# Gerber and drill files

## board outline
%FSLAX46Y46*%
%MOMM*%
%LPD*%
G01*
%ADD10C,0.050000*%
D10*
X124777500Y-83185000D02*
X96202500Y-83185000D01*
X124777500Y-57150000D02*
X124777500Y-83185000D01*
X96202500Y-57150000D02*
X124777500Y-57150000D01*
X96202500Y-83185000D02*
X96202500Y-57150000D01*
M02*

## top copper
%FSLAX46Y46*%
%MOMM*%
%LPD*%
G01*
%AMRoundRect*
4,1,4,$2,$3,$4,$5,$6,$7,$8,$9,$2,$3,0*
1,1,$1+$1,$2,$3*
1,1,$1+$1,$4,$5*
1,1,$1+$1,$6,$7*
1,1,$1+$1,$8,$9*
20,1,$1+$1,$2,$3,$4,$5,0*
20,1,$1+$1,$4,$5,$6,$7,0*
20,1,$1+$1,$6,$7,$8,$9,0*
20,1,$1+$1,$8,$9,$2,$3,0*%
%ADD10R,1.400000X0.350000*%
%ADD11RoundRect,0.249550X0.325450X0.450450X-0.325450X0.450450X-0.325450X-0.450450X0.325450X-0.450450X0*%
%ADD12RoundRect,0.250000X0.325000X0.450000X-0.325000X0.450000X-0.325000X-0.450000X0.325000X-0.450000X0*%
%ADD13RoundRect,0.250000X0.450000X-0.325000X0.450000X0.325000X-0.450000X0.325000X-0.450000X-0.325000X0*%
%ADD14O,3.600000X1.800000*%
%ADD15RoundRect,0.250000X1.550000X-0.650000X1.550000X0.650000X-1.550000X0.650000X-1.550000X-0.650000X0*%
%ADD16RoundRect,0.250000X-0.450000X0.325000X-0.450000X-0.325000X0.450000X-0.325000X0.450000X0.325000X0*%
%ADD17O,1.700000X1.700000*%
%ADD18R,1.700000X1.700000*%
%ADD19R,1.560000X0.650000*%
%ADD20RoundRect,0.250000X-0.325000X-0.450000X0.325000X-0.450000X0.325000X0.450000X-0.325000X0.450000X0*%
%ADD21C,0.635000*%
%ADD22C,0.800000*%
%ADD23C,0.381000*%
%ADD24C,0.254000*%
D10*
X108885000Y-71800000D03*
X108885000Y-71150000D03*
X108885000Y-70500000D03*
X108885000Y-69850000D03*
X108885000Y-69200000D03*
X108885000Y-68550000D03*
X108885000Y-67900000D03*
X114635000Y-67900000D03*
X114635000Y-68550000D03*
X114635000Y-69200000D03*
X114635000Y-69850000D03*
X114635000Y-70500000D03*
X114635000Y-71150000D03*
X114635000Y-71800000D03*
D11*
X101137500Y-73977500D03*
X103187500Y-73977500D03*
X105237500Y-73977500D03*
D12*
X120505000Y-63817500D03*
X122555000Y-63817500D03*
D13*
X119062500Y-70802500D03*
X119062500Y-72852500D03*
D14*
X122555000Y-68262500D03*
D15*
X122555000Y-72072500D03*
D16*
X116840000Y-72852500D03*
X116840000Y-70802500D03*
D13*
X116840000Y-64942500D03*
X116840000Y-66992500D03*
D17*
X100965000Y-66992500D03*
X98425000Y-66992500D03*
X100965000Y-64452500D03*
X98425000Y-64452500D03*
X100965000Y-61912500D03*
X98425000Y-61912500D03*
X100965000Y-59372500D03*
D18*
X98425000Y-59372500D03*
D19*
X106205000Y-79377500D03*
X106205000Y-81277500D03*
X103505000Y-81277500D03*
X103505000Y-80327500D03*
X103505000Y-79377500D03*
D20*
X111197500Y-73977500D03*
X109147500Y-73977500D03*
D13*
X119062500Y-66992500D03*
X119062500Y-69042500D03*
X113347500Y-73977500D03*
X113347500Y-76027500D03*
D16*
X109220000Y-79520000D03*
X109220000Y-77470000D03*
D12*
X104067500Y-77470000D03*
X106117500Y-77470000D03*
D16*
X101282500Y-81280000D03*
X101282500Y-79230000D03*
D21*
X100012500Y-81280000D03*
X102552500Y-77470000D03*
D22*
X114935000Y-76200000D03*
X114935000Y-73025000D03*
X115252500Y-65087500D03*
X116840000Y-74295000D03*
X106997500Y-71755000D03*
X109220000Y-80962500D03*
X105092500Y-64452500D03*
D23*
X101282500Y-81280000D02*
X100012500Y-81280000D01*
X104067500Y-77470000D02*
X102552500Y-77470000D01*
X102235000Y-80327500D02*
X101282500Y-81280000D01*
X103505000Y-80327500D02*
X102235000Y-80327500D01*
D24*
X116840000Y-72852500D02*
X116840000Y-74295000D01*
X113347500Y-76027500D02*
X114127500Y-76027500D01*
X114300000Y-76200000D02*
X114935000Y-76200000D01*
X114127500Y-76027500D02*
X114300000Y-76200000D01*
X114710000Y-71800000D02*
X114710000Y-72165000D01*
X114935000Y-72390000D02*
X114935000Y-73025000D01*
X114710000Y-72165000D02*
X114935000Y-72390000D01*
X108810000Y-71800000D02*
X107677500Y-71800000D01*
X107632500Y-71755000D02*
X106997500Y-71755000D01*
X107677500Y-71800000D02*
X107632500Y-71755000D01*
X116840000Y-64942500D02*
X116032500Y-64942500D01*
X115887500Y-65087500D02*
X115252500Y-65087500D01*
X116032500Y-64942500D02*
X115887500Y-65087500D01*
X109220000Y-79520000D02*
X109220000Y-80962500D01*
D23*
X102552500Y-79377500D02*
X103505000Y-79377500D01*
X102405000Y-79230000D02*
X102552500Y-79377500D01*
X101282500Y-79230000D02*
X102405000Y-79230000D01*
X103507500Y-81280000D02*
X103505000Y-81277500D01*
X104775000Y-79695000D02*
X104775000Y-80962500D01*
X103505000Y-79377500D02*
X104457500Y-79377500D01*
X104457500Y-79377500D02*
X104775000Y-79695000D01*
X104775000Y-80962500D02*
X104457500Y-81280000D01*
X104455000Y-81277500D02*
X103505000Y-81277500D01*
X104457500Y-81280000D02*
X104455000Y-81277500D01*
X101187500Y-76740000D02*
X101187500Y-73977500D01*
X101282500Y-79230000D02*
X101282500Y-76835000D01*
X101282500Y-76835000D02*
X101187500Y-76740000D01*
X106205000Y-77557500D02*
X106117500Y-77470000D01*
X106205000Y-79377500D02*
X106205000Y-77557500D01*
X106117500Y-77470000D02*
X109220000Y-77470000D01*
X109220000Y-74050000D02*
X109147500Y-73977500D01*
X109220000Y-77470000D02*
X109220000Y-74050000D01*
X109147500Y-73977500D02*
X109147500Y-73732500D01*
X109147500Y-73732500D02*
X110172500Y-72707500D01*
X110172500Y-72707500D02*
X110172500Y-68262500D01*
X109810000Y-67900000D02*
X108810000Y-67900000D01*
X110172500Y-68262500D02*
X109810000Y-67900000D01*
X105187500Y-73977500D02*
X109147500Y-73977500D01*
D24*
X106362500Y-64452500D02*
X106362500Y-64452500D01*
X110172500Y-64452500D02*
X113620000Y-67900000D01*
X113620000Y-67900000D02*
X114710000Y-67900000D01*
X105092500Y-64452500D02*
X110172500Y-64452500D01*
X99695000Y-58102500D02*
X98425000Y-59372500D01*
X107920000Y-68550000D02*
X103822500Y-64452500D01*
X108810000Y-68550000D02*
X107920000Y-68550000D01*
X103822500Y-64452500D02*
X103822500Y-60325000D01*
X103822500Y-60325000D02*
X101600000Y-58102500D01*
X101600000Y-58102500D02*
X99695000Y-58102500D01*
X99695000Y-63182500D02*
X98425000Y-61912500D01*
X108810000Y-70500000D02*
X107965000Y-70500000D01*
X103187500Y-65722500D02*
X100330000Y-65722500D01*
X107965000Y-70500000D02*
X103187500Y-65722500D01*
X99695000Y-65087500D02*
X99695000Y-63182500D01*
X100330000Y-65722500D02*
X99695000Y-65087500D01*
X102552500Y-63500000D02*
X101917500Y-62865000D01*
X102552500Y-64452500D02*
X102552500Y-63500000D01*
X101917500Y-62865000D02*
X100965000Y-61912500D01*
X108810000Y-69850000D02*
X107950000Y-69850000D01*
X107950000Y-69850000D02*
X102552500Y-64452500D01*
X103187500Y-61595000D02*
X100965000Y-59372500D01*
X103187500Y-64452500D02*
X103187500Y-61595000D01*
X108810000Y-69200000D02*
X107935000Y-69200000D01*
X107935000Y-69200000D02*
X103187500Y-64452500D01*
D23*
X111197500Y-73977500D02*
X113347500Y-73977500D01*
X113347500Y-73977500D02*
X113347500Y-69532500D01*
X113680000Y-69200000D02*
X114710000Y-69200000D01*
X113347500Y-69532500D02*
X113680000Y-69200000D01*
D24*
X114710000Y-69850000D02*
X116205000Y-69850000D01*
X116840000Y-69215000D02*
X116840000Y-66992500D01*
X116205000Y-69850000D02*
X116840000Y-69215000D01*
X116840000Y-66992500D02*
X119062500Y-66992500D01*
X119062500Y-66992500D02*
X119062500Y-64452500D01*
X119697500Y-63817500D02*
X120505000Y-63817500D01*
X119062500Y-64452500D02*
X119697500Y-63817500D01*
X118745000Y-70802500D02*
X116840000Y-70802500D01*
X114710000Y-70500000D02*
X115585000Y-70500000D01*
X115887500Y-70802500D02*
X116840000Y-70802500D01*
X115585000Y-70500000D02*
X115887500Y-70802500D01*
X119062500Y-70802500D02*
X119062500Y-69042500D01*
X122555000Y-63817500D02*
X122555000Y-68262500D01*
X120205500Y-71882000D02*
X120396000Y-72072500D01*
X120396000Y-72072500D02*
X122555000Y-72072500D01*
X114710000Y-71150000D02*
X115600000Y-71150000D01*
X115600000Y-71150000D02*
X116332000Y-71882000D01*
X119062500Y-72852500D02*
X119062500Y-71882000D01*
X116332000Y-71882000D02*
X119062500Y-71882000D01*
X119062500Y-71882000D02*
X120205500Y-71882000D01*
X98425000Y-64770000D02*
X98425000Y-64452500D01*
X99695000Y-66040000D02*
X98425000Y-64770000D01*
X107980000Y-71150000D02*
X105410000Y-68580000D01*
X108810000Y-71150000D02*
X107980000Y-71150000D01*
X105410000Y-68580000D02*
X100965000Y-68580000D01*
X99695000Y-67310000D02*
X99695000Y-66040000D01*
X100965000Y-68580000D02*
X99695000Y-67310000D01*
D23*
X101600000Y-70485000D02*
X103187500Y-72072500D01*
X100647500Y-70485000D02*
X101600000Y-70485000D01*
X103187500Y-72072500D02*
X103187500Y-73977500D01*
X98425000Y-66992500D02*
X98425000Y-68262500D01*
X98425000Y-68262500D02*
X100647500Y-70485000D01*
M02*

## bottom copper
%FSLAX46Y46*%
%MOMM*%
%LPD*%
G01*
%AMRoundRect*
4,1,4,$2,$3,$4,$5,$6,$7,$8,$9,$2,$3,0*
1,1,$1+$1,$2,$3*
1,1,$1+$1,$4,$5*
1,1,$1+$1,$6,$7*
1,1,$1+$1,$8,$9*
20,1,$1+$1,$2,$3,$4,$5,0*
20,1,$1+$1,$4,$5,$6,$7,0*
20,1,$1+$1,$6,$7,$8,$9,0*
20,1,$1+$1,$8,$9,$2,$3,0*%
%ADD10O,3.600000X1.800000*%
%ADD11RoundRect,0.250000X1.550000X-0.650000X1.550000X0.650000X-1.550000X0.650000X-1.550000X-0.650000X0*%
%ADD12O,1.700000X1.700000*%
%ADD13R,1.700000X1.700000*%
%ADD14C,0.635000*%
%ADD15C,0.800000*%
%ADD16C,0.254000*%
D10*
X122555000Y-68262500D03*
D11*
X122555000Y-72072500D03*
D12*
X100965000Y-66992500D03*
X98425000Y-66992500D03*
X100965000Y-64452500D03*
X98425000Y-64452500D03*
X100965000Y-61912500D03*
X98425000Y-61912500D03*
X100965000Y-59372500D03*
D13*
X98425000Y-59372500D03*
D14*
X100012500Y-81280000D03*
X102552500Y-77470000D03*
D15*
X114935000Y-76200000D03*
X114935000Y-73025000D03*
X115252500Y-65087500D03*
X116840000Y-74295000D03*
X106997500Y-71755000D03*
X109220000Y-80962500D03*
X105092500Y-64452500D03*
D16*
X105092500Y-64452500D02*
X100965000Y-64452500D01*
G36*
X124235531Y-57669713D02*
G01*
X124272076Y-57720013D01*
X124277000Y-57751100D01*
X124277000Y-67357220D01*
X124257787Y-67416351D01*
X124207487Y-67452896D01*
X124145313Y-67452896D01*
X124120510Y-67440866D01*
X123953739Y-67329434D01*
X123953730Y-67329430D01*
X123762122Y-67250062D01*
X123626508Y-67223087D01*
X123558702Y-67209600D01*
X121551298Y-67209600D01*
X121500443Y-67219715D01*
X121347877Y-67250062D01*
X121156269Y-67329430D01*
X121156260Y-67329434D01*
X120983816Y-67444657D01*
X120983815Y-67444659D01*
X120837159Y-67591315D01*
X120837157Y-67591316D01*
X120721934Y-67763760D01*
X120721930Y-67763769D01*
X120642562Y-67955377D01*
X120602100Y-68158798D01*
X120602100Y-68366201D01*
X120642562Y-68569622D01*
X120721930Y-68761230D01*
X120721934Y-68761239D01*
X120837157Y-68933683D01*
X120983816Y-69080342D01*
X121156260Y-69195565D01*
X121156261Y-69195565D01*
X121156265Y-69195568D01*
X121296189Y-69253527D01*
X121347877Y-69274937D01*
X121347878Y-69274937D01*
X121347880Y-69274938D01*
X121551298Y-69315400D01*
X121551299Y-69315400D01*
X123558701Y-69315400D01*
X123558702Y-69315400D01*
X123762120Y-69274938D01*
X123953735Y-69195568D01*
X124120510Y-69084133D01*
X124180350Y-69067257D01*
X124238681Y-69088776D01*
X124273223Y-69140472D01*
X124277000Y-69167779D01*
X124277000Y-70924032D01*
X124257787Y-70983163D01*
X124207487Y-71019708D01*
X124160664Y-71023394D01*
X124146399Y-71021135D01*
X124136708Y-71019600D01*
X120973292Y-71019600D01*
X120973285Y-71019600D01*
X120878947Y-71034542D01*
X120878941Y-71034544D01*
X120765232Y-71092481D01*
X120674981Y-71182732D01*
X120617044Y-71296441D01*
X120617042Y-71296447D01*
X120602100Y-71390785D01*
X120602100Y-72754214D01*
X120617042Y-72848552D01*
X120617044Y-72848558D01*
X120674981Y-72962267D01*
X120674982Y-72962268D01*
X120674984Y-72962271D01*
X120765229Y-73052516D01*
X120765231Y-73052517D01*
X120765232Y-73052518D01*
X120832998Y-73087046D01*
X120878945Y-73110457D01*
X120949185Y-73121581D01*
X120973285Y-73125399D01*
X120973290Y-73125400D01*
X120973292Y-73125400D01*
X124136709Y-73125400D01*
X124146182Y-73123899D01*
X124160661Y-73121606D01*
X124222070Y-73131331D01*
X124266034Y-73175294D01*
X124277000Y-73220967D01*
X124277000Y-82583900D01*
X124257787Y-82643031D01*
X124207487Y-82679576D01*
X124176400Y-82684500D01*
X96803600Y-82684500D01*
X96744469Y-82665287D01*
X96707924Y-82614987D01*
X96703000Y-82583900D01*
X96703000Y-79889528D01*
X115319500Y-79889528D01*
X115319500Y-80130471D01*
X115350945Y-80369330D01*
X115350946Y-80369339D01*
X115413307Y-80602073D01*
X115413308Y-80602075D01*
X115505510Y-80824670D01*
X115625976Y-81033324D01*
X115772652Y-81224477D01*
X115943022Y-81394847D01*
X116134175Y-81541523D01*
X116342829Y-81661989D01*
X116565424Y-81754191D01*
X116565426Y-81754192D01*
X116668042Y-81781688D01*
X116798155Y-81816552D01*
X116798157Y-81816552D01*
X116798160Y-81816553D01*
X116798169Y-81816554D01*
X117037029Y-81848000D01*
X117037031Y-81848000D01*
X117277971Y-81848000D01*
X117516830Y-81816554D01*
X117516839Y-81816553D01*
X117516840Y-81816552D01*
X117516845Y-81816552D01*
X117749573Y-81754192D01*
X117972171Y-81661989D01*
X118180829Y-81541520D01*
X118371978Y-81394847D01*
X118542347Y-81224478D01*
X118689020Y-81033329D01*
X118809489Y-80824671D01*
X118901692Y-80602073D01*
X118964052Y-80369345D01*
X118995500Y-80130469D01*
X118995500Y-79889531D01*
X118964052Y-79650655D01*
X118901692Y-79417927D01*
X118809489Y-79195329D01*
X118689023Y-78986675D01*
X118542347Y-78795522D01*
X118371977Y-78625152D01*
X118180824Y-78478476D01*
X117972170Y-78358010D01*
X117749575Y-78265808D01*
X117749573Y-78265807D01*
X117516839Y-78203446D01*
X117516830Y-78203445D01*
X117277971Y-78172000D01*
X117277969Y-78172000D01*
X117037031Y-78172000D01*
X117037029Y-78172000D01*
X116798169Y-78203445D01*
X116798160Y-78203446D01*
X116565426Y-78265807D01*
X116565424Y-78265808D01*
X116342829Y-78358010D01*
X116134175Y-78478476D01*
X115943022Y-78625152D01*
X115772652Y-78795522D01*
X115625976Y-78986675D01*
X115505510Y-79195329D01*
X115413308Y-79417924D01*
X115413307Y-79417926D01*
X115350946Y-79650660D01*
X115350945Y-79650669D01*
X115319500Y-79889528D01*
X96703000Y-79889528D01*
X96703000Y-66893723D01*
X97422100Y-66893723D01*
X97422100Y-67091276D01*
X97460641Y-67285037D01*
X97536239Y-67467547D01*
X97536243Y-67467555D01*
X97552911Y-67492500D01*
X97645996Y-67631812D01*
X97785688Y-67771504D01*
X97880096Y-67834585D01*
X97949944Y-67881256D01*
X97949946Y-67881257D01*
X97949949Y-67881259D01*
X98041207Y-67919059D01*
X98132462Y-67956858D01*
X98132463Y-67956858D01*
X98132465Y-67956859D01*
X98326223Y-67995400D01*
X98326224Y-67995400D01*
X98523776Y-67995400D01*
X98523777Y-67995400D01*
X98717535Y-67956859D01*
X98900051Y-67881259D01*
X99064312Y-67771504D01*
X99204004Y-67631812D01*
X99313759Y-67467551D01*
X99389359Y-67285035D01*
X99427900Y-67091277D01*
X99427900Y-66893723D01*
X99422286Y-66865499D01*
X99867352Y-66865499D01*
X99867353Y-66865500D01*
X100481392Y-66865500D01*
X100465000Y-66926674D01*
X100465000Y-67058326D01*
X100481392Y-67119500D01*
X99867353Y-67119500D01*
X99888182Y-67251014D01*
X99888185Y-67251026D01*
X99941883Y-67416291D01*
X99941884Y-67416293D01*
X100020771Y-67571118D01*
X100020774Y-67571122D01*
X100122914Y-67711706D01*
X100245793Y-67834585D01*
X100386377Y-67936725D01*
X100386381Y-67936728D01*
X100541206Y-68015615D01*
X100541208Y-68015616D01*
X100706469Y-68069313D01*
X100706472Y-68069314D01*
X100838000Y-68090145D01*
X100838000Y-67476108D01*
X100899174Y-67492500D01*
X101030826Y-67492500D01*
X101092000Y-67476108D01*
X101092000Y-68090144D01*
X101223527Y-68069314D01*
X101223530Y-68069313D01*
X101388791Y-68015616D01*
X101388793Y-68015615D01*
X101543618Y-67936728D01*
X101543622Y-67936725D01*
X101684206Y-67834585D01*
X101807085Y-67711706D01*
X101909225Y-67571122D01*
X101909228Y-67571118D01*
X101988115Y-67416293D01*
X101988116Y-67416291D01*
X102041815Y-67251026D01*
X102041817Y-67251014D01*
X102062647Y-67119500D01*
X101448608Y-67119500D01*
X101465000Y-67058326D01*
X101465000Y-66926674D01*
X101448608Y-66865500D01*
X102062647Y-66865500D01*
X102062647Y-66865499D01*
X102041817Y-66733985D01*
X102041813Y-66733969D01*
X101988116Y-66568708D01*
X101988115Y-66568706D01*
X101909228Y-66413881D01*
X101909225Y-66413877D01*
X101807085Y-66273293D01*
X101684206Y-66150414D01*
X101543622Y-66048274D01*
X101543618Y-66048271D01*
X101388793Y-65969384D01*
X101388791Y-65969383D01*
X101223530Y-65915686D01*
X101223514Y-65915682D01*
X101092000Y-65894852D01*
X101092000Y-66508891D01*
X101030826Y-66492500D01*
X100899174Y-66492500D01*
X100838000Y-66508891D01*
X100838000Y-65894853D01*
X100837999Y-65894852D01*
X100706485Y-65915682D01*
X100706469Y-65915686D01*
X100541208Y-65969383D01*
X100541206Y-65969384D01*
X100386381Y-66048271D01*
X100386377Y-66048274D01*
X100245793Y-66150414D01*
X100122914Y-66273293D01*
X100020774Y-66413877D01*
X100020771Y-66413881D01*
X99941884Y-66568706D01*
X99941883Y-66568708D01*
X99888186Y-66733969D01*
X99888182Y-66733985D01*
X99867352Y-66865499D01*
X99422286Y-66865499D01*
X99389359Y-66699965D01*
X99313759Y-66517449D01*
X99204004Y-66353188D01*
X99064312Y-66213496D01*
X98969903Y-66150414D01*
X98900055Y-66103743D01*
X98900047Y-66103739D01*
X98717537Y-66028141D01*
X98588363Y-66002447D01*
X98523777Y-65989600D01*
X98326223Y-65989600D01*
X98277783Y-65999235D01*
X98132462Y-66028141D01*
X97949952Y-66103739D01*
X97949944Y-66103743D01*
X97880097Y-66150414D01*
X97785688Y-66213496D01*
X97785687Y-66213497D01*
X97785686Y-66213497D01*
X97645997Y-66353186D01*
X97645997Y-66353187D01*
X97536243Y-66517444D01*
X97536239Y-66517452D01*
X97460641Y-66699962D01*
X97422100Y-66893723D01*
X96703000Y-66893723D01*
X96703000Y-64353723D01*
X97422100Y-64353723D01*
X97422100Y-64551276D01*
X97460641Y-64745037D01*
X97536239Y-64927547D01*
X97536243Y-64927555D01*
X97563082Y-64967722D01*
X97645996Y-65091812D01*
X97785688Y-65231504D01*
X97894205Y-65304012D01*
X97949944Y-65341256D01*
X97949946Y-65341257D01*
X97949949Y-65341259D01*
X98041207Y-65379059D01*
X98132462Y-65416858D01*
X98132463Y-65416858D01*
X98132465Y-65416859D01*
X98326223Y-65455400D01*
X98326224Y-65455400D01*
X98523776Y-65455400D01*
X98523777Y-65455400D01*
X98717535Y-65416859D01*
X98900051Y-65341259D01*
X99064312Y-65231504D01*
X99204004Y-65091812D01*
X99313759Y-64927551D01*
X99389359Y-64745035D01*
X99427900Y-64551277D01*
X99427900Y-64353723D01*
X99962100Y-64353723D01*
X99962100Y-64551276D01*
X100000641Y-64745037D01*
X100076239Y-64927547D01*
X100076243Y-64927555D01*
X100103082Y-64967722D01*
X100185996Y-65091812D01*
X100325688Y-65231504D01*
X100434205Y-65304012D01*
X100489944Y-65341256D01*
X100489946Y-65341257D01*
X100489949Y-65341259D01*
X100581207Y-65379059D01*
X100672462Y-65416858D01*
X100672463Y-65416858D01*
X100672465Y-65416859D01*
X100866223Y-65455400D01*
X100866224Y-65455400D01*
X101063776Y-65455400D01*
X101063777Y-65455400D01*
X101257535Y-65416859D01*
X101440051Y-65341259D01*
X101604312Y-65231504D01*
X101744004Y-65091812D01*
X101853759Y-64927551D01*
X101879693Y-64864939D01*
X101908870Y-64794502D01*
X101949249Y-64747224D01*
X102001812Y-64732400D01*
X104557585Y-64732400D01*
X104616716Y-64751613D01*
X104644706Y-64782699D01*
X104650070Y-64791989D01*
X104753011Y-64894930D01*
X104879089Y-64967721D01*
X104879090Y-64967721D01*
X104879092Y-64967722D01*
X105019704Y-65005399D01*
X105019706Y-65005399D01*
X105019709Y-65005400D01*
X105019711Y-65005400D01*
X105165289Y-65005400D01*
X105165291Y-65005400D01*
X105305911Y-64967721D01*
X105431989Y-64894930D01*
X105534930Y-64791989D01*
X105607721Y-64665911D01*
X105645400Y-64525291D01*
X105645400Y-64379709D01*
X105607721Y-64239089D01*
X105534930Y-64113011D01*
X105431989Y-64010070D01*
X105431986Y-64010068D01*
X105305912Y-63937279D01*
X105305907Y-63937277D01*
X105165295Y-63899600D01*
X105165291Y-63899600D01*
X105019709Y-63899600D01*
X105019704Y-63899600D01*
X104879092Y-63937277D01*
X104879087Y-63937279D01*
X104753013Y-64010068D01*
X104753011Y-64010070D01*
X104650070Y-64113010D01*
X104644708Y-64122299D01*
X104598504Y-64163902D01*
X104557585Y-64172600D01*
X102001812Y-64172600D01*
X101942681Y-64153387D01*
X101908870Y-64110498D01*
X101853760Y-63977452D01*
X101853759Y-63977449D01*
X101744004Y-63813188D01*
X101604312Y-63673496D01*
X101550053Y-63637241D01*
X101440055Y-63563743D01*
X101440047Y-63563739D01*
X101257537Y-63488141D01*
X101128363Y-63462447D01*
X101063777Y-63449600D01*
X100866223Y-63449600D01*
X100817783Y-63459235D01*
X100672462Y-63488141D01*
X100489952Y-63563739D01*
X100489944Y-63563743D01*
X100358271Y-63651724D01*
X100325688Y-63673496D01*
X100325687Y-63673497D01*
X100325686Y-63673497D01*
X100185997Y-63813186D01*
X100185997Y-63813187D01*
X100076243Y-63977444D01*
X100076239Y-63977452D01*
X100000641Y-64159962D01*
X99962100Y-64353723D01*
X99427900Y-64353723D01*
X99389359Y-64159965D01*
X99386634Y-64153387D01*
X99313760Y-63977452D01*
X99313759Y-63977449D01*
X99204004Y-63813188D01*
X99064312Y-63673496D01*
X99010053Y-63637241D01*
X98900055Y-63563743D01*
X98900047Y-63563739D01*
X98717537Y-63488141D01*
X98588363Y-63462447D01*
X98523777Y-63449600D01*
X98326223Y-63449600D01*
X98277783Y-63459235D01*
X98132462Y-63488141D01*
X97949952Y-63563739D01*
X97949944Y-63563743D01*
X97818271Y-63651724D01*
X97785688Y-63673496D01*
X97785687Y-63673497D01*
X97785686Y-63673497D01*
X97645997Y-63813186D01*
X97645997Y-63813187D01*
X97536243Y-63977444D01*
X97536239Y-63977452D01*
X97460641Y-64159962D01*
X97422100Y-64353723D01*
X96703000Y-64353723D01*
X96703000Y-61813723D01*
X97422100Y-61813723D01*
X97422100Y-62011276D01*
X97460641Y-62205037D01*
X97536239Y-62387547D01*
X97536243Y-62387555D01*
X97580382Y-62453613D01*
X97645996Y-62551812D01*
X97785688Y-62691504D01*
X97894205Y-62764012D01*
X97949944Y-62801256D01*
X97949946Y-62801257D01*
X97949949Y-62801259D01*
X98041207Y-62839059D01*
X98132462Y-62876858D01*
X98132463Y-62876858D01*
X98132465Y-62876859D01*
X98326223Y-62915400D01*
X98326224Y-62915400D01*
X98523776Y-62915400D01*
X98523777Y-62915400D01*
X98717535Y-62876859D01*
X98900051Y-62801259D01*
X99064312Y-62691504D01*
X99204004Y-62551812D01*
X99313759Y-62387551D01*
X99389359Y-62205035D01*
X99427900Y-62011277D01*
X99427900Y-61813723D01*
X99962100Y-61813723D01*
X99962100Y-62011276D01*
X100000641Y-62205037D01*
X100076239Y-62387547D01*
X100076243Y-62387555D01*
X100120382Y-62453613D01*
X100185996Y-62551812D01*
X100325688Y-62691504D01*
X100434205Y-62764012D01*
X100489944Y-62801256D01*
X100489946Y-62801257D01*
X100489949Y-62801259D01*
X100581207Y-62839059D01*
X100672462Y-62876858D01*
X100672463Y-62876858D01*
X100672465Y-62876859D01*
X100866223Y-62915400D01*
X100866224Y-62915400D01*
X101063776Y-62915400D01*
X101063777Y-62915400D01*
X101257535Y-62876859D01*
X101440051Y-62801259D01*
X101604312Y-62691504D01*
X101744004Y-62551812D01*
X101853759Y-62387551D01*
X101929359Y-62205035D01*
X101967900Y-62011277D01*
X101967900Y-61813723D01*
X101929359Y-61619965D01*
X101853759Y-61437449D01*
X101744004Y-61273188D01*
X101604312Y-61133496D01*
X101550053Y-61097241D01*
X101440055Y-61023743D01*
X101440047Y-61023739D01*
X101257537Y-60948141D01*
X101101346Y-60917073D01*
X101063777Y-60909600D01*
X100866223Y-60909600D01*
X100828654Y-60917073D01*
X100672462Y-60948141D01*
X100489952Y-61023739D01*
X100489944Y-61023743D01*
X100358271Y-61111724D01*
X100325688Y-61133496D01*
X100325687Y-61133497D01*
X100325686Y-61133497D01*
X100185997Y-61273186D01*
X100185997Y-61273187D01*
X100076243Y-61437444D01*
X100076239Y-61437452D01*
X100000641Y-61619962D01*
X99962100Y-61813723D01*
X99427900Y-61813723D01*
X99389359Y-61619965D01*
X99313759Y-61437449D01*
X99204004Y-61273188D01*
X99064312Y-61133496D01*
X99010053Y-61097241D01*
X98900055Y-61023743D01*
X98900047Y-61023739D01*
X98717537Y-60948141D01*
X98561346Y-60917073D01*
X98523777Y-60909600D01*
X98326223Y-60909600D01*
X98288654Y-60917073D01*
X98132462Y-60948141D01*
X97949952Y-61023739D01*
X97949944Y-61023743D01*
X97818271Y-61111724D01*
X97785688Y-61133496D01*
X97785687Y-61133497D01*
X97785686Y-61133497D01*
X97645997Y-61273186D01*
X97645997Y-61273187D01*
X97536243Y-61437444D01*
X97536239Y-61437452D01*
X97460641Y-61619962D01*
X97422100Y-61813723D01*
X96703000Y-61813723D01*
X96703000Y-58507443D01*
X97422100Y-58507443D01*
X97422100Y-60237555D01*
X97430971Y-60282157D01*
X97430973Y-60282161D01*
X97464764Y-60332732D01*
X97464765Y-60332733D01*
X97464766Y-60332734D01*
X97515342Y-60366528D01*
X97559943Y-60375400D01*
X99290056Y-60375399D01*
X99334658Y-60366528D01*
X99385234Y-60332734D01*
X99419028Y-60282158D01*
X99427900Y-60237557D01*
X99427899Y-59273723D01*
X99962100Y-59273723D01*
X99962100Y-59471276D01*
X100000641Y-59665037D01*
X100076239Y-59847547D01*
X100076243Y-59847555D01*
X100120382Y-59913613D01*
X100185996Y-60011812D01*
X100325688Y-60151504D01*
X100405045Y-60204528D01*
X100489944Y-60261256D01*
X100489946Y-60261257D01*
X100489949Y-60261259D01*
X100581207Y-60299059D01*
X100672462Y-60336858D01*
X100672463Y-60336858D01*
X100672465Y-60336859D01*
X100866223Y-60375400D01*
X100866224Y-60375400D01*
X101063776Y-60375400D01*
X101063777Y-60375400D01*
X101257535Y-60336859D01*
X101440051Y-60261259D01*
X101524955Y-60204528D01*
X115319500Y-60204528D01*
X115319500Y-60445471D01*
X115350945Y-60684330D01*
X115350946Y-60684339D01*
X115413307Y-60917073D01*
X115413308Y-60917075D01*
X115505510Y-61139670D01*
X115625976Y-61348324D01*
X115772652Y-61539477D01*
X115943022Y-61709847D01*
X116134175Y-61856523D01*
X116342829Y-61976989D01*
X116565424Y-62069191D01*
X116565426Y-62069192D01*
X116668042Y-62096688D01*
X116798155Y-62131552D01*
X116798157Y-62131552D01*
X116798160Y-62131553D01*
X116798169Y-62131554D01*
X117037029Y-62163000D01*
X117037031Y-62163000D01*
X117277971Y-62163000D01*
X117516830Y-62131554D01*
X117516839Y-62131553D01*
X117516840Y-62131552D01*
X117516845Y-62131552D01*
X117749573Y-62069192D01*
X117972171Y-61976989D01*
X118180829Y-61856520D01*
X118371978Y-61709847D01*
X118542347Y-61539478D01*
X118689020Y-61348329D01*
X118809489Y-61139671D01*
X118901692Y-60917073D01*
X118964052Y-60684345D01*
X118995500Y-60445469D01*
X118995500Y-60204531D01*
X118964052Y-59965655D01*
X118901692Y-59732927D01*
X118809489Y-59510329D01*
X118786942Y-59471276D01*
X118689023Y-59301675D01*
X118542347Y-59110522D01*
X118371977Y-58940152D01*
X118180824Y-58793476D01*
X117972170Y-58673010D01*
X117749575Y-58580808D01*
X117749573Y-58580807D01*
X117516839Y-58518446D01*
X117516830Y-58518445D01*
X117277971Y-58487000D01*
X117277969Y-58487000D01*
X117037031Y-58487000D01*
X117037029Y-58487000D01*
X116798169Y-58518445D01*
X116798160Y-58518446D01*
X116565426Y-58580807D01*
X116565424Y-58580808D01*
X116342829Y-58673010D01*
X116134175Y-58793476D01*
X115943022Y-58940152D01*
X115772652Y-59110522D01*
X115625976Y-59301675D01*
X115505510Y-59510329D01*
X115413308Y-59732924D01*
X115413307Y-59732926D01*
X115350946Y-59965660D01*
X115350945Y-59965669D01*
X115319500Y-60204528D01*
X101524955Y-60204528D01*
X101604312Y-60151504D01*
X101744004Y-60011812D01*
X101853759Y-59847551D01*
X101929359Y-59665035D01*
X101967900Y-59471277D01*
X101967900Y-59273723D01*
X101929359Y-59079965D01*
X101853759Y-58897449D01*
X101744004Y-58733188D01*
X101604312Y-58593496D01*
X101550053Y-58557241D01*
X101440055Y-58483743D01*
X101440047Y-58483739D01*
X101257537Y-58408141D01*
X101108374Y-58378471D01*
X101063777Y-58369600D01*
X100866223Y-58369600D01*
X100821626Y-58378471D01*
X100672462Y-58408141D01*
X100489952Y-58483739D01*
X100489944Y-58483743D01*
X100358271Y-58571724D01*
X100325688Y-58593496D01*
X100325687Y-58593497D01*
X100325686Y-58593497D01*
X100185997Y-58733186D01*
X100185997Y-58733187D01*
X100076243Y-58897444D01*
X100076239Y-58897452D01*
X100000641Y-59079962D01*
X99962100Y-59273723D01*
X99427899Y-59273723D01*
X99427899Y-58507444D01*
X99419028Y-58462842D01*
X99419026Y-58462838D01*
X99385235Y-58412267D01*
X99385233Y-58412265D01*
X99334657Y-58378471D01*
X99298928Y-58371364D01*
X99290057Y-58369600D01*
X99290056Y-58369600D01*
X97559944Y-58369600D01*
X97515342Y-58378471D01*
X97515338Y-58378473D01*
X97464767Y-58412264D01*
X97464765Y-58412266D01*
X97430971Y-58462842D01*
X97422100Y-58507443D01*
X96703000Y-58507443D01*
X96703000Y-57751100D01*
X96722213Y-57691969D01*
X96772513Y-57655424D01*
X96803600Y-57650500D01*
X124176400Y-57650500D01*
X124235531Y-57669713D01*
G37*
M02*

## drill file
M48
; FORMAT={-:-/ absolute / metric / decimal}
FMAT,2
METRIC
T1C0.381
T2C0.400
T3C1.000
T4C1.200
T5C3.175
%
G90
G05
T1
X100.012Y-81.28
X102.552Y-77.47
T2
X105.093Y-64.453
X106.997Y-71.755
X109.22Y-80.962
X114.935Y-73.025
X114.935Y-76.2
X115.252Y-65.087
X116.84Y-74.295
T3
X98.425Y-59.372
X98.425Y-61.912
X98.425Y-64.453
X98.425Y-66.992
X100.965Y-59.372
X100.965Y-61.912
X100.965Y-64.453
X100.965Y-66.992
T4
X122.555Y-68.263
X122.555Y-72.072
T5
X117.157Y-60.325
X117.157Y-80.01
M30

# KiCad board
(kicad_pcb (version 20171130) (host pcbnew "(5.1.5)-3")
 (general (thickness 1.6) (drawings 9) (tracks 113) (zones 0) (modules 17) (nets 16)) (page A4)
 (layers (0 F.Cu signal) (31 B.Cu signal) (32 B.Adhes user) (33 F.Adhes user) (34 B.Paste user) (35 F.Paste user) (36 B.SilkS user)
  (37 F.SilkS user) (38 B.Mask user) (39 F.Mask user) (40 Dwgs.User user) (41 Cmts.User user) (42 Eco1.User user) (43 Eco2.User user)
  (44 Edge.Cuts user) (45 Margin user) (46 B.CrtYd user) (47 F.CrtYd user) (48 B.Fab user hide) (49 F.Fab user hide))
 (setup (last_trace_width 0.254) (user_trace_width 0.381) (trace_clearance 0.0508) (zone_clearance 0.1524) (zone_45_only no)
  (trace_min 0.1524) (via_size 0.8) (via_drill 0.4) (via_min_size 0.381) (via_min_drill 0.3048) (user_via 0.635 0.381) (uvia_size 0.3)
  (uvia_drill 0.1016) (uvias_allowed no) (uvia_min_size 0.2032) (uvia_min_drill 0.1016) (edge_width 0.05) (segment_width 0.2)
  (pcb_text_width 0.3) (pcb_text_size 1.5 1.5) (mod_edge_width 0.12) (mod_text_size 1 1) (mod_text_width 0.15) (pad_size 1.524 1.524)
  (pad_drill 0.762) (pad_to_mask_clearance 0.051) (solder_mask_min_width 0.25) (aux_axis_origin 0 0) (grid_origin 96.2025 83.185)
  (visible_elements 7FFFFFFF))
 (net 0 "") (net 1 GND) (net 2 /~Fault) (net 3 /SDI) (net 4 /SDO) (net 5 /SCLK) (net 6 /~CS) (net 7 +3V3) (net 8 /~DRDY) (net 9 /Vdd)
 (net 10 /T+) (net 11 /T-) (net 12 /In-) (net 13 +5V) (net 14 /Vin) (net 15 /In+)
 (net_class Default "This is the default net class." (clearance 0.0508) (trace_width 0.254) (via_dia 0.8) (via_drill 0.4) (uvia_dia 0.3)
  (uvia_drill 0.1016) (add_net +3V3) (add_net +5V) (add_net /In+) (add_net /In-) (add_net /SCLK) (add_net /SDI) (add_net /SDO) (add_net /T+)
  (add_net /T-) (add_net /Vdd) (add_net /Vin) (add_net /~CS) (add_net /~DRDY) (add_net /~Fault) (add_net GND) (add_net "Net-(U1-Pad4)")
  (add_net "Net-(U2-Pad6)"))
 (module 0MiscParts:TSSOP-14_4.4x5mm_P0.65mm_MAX (layer F.Cu) (at 111.76 69.85 180)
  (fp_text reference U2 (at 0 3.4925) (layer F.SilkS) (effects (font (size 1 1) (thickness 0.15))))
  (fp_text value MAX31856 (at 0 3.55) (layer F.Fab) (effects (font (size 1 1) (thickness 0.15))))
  (pad 14 smd rect (at 2.875 -1.95 180) (size 1.4 0.35) (layers F.Cu F.Paste F.Mask) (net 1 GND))
  (pad 13 smd rect (at 2.875 -1.3 180) (size 1.4 0.35) (layers F.Cu F.Paste F.Mask) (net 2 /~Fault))
  (pad 12 smd rect (at 2.875 -0.65 180) (size 1.4 0.35) (layers F.Cu F.Paste F.Mask) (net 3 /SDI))
  (pad 11 smd rect (at 2.875 0 180) (size 1.4 0.35) (layers F.Cu F.Paste F.Mask) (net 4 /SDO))
  (pad 10 smd rect (at 2.875 0.65 180) (size 1.4 0.35) (layers F.Cu F.Paste F.Mask) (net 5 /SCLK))
  (pad 9 smd rect (at 2.875 1.3 180) (size 1.4 0.35) (layers F.Cu F.Paste F.Mask) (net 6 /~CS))
  (pad 8 smd rect (at 2.875 1.95 180) (size 1.4 0.35) (layers F.Cu F.Paste F.Mask) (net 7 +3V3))
  (pad 7 smd rect (at -2.875 1.95 180) (size 1.4 0.35) (layers F.Cu F.Paste F.Mask) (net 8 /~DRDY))
  (pad 6 smd rect (at -2.875 1.3 180) (size 1.4 0.35) (layers F.Cu F.Paste F.Mask))
  (pad 5 smd rect (at -2.875 0.65 180) (size 1.4 0.35) (layers F.Cu F.Paste F.Mask) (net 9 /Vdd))
  (pad 4 smd rect (at -2.875 0 180) (size 1.4 0.35) (layers F.Cu F.Paste F.Mask) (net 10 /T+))
  (pad 3 smd rect (at -2.875 -0.65 180) (size 1.4 0.35) (layers F.Cu F.Paste F.Mask) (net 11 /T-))
  (pad 2 smd rect (at -2.875 -1.3 180) (size 1.4 0.35) (layers F.Cu F.Paste F.Mask) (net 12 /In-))
  (pad 1 smd rect (at -2.875 -1.95 180) (size 1.4 0.35) (layers F.Cu F.Paste F.Mask) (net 1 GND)))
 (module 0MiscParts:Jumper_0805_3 (layer F.Cu) (at 103.1875 73.9775 180)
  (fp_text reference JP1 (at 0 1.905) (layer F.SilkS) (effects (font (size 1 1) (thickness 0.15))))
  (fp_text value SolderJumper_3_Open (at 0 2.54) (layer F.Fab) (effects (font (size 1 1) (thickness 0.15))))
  (pad 3 smd roundrect (at 2.05 0 180) (size 1.15 1.4) (layers F.Cu F.Paste F.Mask) (roundrect_rratio 0.217) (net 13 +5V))
  (pad 2 smd roundrect (at 0 0 180) (size 1.15 1.4) (layers F.Cu F.Paste F.Mask) (roundrect_rratio 0.217) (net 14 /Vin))
  (pad 1 smd roundrect (at -2.05 0 180) (size 1.15 1.4) (layers F.Cu F.Paste F.Mask) (roundrect_rratio 0.217) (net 7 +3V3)))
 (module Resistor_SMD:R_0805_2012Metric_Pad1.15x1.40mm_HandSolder (layer F.Cu) (at 121.53 63.8175 180)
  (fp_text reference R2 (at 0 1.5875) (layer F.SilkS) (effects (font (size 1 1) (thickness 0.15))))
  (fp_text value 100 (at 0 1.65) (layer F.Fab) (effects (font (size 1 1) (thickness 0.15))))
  (pad 2 smd roundrect (at 1.025 0 180) (size 1.15 1.4) (layers F.Cu F.Paste F.Mask) (roundrect_rratio 0.217391) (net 10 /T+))
  (pad 1 smd roundrect (at -1.025 0 180) (size 1.15 1.4) (layers F.Cu F.Paste F.Mask) (roundrect_rratio 0.217391) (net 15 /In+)))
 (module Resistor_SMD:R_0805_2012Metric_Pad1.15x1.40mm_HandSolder (layer F.Cu) (at 119.0625 71.8275 90)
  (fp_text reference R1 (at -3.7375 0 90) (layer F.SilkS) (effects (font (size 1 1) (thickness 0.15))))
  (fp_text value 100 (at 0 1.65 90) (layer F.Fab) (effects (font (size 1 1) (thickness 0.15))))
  (pad 2 smd roundrect (at 1.025 0 90) (size 1.15 1.4) (layers F.Cu F.Paste F.Mask) (roundrect_rratio 0.217391) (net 11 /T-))
  (pad 1 smd roundrect (at -1.025 0 90) (size 1.15 1.4) (layers F.Cu F.Paste F.Mask) (roundrect_rratio 0.217391) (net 12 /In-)))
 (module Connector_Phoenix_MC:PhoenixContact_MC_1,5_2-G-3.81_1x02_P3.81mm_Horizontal (layer F.Cu) (at 122.555 72.0725 90)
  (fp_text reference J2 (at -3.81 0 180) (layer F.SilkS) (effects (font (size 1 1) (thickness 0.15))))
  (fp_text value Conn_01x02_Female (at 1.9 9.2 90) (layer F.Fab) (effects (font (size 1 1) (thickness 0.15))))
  (pad 2 thru_hole oval (at 3.81 0 90) (size 1.8 3.6) (drill 1.2) (layers *.Cu *.Mask) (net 15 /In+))
  (pad 1 thru_hole roundrect (at 0 0 90) (size 1.8 3.6) (drill 1.2) (layers *.Cu *.Mask) (roundrect_rratio 0.138889) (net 12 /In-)))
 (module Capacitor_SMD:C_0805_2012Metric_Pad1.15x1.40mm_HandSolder (layer F.Cu) (at 116.84 71.8275 270)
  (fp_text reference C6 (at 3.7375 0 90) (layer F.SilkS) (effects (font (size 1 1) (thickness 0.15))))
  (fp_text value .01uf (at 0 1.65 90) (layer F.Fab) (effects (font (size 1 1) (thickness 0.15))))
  (pad 2 smd roundrect (at 1.025 0 270) (size 1.15 1.4) (layers F.Cu F.Paste F.Mask) (roundrect_rratio 0.217391) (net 1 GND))
  (pad 1 smd roundrect (at -1.025 0 270) (size 1.15 1.4) (layers F.Cu F.Paste F.Mask) (roundrect_rratio 0.217391) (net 11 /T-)))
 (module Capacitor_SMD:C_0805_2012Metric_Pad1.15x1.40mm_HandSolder (layer F.Cu) (at 116.84 65.9675 90)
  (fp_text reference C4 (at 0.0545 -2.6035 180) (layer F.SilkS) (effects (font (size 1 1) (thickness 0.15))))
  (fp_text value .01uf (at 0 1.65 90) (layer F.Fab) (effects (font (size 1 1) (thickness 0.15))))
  (pad 2 smd roundrect (at 1.025 0 90) (size 1.15 1.4) (layers F.Cu F.Paste F.Mask) (roundrect_rratio 0.217391) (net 1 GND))
  (pad 1 smd roundrect (at -1.025 0 90) (size 1.15 1.4) (layers F.Cu F.Paste F.Mask) (roundrect_rratio 0.217391) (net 10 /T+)))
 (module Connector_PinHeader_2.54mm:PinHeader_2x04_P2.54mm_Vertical (layer F.Cu) (at 98.425 59.3725)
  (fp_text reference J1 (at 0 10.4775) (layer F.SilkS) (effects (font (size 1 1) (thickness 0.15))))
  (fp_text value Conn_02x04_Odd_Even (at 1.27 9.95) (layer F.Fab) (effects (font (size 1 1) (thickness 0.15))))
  (pad 8 thru_hole oval (at 2.54 7.62) (size 1.7 1.7) (drill 1) (layers *.Cu *.Mask) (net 1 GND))
  (pad 7 thru_hole oval (at 0 7.62) (size 1.7 1.7) (drill 1) (layers *.Cu *.Mask) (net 14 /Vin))
  (pad 6 thru_hole oval (at 2.54 5.08) (size 1.7 1.7) (drill 1) (layers *.Cu *.Mask) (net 8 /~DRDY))
  (pad 5 thru_hole oval (at 0 5.08) (size 1.7 1.7) (drill 1) (layers *.Cu *.Mask) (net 2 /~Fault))
  (pad 4 thru_hole oval (at 2.54 2.54) (size 1.7 1.7) (drill 1) (layers *.Cu *.Mask) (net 4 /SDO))
  (pad 3 thru_hole oval (at 0 2.54) (size 1.7 1.7) (drill 1) (layers *.Cu *.Mask) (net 3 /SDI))
  (pad 2 thru_hole oval (at 2.54 0) (size 1.7 1.7) (drill 1) (layers *.Cu *.Mask) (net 5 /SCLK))
  (pad 1 thru_hole rect (at 0 0) (size 1.7 1.7) (drill 1) (layers *.Cu *.Mask) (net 6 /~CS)))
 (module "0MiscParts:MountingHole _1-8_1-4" (layer F.Cu) (at 117.1575 80.01)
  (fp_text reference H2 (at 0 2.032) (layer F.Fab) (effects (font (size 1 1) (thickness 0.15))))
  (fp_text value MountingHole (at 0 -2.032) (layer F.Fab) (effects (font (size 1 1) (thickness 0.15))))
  (pad "" np_thru_hole circle (at 0 0) (size 3.175 3.175) (drill 3.175) (layers *.Cu *.Mask)))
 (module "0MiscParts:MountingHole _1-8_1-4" (layer F.Cu) (at 117.1575 60.325)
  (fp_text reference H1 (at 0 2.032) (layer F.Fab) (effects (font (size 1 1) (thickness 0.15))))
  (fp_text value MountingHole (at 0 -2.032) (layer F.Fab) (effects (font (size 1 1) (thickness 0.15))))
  (pad "" np_thru_hole circle (at 0 0) (size 3.175 3.175) (drill 3.175) (layers *.Cu *.Mask)))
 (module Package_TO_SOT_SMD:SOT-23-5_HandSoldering (layer F.Cu) (at 104.855 80.3275)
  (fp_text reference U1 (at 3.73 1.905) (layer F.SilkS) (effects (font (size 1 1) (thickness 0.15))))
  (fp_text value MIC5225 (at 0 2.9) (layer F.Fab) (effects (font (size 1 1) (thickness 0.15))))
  (pad 5 smd rect (at 1.35 -0.95) (size 1.56 0.65) (layers F.Cu F.Paste F.Mask) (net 7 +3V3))
  (pad 4 smd rect (at 1.35 0.95) (size 1.56 0.65) (layers F.Cu F.Paste F.Mask))
  (pad 3 smd rect (at -1.35 0.95) (size 1.56 0.65) (layers F.Cu F.Paste F.Mask) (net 13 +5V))
  (pad 2 smd rect (at -1.35 0) (size 1.56 0.65) (layers F.Cu F.Paste F.Mask) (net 1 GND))
  (pad 1 smd rect (at -1.35 -0.95) (size 1.56 0.65) (layers F.Cu F.Paste F.Mask) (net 13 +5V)))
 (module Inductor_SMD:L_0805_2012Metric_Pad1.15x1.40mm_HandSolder (layer F.Cu) (at 110.1725 73.9775)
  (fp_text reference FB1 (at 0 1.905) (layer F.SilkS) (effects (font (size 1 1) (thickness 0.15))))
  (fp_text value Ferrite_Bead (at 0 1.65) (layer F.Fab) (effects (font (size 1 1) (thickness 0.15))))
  (pad 2 smd roundrect (at 1.025 0) (size 1.15 1.4) (layers F.Cu F.Paste F.Mask) (roundrect_rratio 0.217391) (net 9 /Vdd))
  (pad 1 smd roundrect (at -1.025 0) (size 1.15 1.4) (layers F.Cu F.Paste F.Mask) (roundrect_rratio 0.217391) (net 7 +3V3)))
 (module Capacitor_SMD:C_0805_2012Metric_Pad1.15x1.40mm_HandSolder (layer F.Cu) (at 119.0625 68.0175 90)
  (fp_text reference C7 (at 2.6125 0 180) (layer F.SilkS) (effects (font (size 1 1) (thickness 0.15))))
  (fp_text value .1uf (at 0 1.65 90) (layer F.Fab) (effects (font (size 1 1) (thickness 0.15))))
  (pad 2 smd roundrect (at 1.025 0 90) (size 1.15 1.4) (layers F.Cu F.Paste F.Mask) (roundrect_rratio 0.217391) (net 10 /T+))
  (pad 1 smd roundrect (at -1.025 0 90) (size 1.15 1.4) (layers F.Cu F.Paste F.Mask) (roundrect_rratio 0.217391) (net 11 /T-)))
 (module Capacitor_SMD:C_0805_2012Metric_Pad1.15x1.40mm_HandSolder (layer F.Cu) (at 113.3475 75.0025 90)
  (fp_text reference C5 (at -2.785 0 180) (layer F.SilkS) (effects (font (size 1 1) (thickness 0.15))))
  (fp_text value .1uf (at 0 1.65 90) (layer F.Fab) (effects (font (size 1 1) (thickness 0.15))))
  (pad 2 smd roundrect (at 1.025 0 90) (size 1.15 1.4) (layers F.Cu F.Paste F.Mask) (roundrect_rratio 0.217391) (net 9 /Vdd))
  (pad 1 smd roundrect (at -1.025 0 90) (size 1.15 1.4) (layers F.Cu F.Paste F.Mask) (roundrect_rratio 0.217391) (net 1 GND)))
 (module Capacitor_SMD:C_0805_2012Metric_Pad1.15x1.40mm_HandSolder (layer F.Cu) (at 109.22 78.495 270)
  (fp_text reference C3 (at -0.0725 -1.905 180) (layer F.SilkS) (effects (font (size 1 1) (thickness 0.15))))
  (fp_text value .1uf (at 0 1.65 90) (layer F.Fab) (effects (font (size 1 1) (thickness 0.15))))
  (pad 2 smd roundrect (at 1.025 0 270) (size 1.15 1.4) (layers F.Cu F.Paste F.Mask) (roundrect_rratio 0.217391) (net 1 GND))
  (pad 1 smd roundrect (at -1.025 0 270) (size 1.15 1.4) (layers F.Cu F.Paste F.Mask) (roundrect_rratio 0.217391) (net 7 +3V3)))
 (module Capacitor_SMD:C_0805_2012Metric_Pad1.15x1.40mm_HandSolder (layer F.Cu) (at 105.0925 77.47 180)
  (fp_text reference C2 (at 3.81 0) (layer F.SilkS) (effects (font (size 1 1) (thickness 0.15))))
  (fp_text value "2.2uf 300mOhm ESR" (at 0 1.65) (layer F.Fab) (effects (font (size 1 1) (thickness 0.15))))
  (pad 2 smd roundrect (at 1.025 0 180) (size 1.15 1.4) (layers F.Cu F.Paste F.Mask) (roundrect_rratio 0.217391) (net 1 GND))
  (pad 1 smd roundrect (at -1.025 0 180) (size 1.15 1.4) (layers F.Cu F.Paste F.Mask) (roundrect_rratio 0.217391) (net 7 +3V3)))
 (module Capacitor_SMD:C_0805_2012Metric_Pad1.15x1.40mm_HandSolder (layer F.Cu) (at 101.2825 80.255 270)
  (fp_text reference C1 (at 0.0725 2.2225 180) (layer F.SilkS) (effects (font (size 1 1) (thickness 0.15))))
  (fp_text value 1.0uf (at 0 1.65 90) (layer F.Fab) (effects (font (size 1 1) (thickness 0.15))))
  (pad 2 smd roundrect (at 1.025 0 270) (size 1.15 1.4) (layers F.Cu F.Paste F.Mask) (roundrect_rratio 0.217391) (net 1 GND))
  (pad 1 smd roundrect (at -1.025 0 270) (size 1.15 1.4) (layers F.Cu F.Paste F.Mask) (roundrect_rratio 0.217391) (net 13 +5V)))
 (gr_line (start 124.7775 83.185) (end 96.2025 83.185) (layer Edge.Cuts) (width 0.05))
 (gr_line (start 124.7775 57.15) (end 124.7775 83.185) (layer Edge.Cuts) (width 0.05))
 (gr_line (start 96.2025 57.15) (end 124.7775 57.15) (layer Edge.Cuts) (width 0.05))
 (gr_line (start 96.2025 83.185) (end 96.2025 57.15) (layer Edge.Cuts) (width 0.05))
 (via (at 100.0125 81.28) (size 0.635) (drill 0.381) (layers F.Cu B.Cu) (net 1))
 (segment (start 101.2825 81.28) (end 100.0125 81.28) (width 0.381) (layer F.Cu) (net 1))
 (via (at 102.5525 77.47) (size 0.635) (drill 0.381) (layers F.Cu B.Cu) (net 1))
 (segment (start 104.0675 77.47) (end 102.5525 77.47) (width 0.381) (layer F.Cu) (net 1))
 (segment (start 102.235 80.3275) (end 101.2825 81.28) (width 0.381) (layer F.Cu) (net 1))
 (segment (start 103.505 80.3275) (end 102.235 80.3275) (width 0.381) (layer F.Cu) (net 1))
 (via (at 114.935 76.2) (size 0.8) (drill 0.4) (layers F.Cu B.Cu) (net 1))
 (via (at 114.935 73.025) (size 0.8) (drill 0.4) (layers F.Cu B.Cu) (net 1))
 (via (at 115.2525 65.0875) (size 0.8) (drill 0.4) (layers F.Cu B.Cu) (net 1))
 (via (at 116.84 74.295) (size 0.8) (drill 0.4) (layers F.Cu B.Cu) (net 1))
 (segment (start 116.84 72.8525) (end 116.84 74.295) (width 0.254) (layer F.Cu) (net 1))
 (segment (start 113.3475 76.0275) (end 114.1275 76.0275) (width 0.254) (layer F.Cu) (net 1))
 (segment (start 114.3 76.2) (end 114.935 76.2) (width 0.254) (layer F.Cu) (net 1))
 (segment (start 114.1275 76.0275) (end 114.3 76.2) (width 0.254) (layer F.Cu) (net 1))
 (segment (start 114.71 71.8) (end 114.71 72.165) (width 0.254) (layer F.Cu) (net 1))
 (segment (start 114.935 72.39) (end 114.935 73.025) (width 0.254) (layer F.Cu) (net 1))
 (segment (start 114.71 72.165) (end 114.935 72.39) (width 0.254) (layer F.Cu) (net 1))
 (via (at 106.9975 71.755) (size 0.8) (drill 0.4) (layers F.Cu B.Cu) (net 1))
 (segment (start 108.81 71.8) (end 107.6775 71.8) (width 0.254) (layer F.Cu) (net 1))
 (segment (start 107.6325 71.755) (end 106.9975 71.755) (width 0.254) (layer F.Cu) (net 1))
 (segment (start 107.6775 71.8) (end 107.6325 71.755) (width 0.254) (layer F.Cu) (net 1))
 (segment (start 116.84 64.9425) (end 116.0325 64.9425) (width 0.254) (layer F.Cu) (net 1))
 (segment (start 115.8875 65.0875) (end 115.2525 65.0875) (width 0.254) (layer F.Cu) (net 1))
 (segment (start 116.0325 64.9425) (end 115.8875 65.0875) (width 0.254) (layer F.Cu) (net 1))
 (via (at 109.22 80.9625) (size 0.8) (drill 0.4) (layers F.Cu B.Cu) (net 1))
 (segment (start 109.22 79.52) (end 109.22 80.9625) (width 0.254) (layer F.Cu) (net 1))
 (segment (start 102.5525 79.3775) (end 103.505 79.3775) (width 0.381) (layer F.Cu) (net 13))
 (segment (start 102.405 79.23) (end 102.5525 79.3775) (width 0.381) (layer F.Cu) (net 13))
 (segment (start 101.2825 79.23) (end 102.405 79.23) (width 0.381) (layer F.Cu) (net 13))
 (segment (start 103.5075 81.28) (end 103.505 81.2775) (width 0.381) (layer F.Cu) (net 13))
 (segment (start 104.775 79.695) (end 104.775 80.9625) (width 0.381) (layer F.Cu) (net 13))
 (segment (start 103.505 79.3775) (end 104.4575 79.3775) (width 0.381) (layer F.Cu) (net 13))
 (segment (start 104.4575 79.3775) (end 104.775 79.695) (width 0.381) (layer F.Cu) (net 13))
 (segment (start 104.775 80.9625) (end 104.4575 81.28) (width 0.381) (layer F.Cu) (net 13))
 (segment (start 104.455 81.2775) (end 103.505 81.2775) (width 0.381) (layer F.Cu) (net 13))
 (segment (start 104.4575 81.28) (end 104.455 81.2775) (width 0.381) (layer F.Cu) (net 13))
 (segment (start 101.1875 76.74) (end 101.1875 73.9775) (width 0.381) (layer F.Cu) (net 13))
 (segment (start 101.2825 79.23) (end 101.2825 76.835) (width 0.381) (layer F.Cu) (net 13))
 (segment (start 101.2825 76.835) (end 101.1875 76.74) (width 0.381) (layer F.Cu) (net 13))
 (segment (start 106.205 77.5575) (end 106.1175 77.47) (width 0.381) (layer F.Cu) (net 7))
 (segment (start 106.205 79.3775) (end 106.205 77.5575) (width 0.381) (layer F.Cu) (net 7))
 (segment (start 106.1175 77.47) (end 109.22 77.47) (width 0.381) (layer F.Cu) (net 7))
 (segment (start 109.22 74.05) (end 109.1475 73.9775) (width 0.381) (layer F.Cu) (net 7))
 (segment (start 109.22 77.47) (end 109.22 74.05) (width 0.381) (layer F.Cu) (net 7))
 (segment (start 109.1475 73.9775) (end 109.1475 73.7325) (width 0.381) (layer F.Cu) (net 7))
 (segment (start 109.1475 73.7325) (end 110.1725 72.7075) (width 0.381) (layer F.Cu) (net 7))
 (segment (start 110.1725 72.7075) (end 110.1725 68.2625) (width 0.381) (layer F.Cu) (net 7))
 (segment (start 109.81 67.9) (end 108.81 67.9) (width 0.381) (layer F.Cu) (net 7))
 (segment (start 110.1725 68.2625) (end 109.81 67.9) (width 0.381) (layer F.Cu) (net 7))
 (segment (start 105.1875 73.9775) (end 109.1475 73.9775) (width 0.381) (layer F.Cu) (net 7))
 (segment (start 106.3625 64.4525) (end 106.3625 64.4525) (width 0.254) (layer F.Cu) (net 8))
 (segment (start 110.1725 64.4525) (end 113.62 67.9) (width 0.254) (layer F.Cu) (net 8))
 (segment (start 113.62 67.9) (end 114.71 67.9) (width 0.254) (layer F.Cu) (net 8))
 (via (at 105.0925 64.4525) (size 0.8) (drill 0.4) (layers F.Cu B.Cu) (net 8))
 (segment (start 105.0925 64.4525) (end 110.1725 64.4525) (width 0.254) (layer F.Cu) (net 8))
 (segment (start 105.0925 64.4525) (end 100.965 64.4525) (width 0.254) (layer B.Cu) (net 8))
 (segment (start 99.695 58.1025) (end 98.425 59.3725) (width 0.254) (layer F.Cu) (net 6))
 (segment (start 107.92 68.55) (end 103.8225 64.4525) (width 0.254) (layer F.Cu) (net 6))
 (segment (start 108.81 68.55) (end 107.92 68.55) (width 0.254) (layer F.Cu) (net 6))
 (segment (start 103.8225 64.4525) (end 103.8225 60.325) (width 0.254) (layer F.Cu) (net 6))
 (segment (start 103.8225 60.325) (end 101.6 58.1025) (width 0.254) (layer F.Cu) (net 6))
 (segment (start 101.6 58.1025) (end 99.695 58.1025) (width 0.254) (layer F.Cu) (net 6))
 (segment (start 99.695 63.1825) (end 98.425 61.9125) (width 0.254) (layer F.Cu) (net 3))
 (segment (start 108.81 70.5) (end 107.965 70.5) (width 0.254) (layer F.Cu) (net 3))
 (segment (start 103.1875 65.7225) (end 100.33 65.7225) (width 0.254) (layer F.Cu) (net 3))
 (segment (start 107.965 70.5) (end 103.1875 65.7225) (width 0.254) (layer F.Cu) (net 3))
 (segment (start 99.695 65.0875) (end 99.695 63.1825) (width 0.254) (layer F.Cu) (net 3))
 (segment (start 100.33 65.7225) (end 99.695 65.0875) (width 0.254) (layer F.Cu) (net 3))
 (segment (start 102.5525 63.5) (end 101.9175 62.865) (width 0.254) (layer F.Cu) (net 4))
 (segment (start 102.5525 64.4525) (end 102.5525 63.5) (width 0.254) (layer F.Cu) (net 4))
 (segment (start 101.9175 62.865) (end 100.965 61.9125) (width 0.254) (layer F.Cu) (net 4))
 (segment (start 108.81 69.85) (end 107.95 69.85) (width 0.254) (layer F.Cu) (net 4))
 (segment (start 107.95 69.85) (end 102.5525 64.4525) (width 0.254) (layer F.Cu) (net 4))
 (segment (start 103.1875 61.595) (end 100.965 59.3725) (width 0.254) (layer F.Cu) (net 5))
 (segment (start 103.1875 64.4525) (end 103.1875 61.595) (width 0.254) (layer F.Cu) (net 5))
 (segment (start 108.81 69.2) (end 107.935 69.2) (width 0.254) (layer F.Cu) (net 5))
 (segment (start 107.935 69.2) (end 103.1875 64.4525) (width 0.254) (layer F.Cu) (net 5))
 (segment (start 111.1975 73.9775) (end 113.3475 73.9775) (width 0.381) (layer F.Cu) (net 9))
 (segment (start 113.3475 73.9775) (end 113.3475 69.5325) (width 0.381) (layer F.Cu) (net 9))
 (segment (start 113.68 69.2) (end 114.71 69.2) (width 0.381) (layer F.Cu) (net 9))
 (segment (start 113.3475 69.5325) (end 113.68 69.2) (width 0.381) (layer F.Cu) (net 9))
 (segment (start 114.71 69.85) (end 116.205 69.85) (width 0.254) (layer F.Cu) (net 10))
 (segment (start 116.84 69.215) (end 116.84 66.9925) (width 0.254) (layer F.Cu) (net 10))
 (segment (start 116.205 69.85) (end 116.84 69.215) (width 0.254) (layer F.Cu) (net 10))
 (segment (start 116.84 66.9925) (end 119.0625 66.9925) (width 0.254) (layer F.Cu) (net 10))
 (segment (start 119.0625 66.9925) (end 119.0625 64.4525) (width 0.254) (layer F.Cu) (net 10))
 (segment (start 119.6975 63.8175) (end 120.505 63.8175) (width 0.254) (layer F.Cu) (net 10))
 (segment (start 119.0625 64.4525) (end 119.6975 63.8175) (width 0.254) (layer F.Cu) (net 10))
 (segment (start 118.745 70.8025) (end 116.84 70.8025) (width 0.254) (layer F.Cu) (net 11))
 (segment (start 114.71 70.5) (end 115.585 70.5) (width 0.254) (layer F.Cu) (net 11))
 (segment (start 115.8875 70.8025) (end 116.84 70.8025) (width 0.254) (layer F.Cu) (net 11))
 (segment (start 115.585 70.5) (end 115.8875 70.8025) (width 0.254) (layer F.Cu) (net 11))
 (segment (start 119.0625 70.8025) (end 119.0625 69.0425) (width 0.254) (layer F.Cu) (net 11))
 (segment (start 122.555 63.8175) (end 122.555 68.2625) (width 0.254) (layer F.Cu) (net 15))
 (segment (start 120.2055 71.882) (end 120.396 72.0725) (width 0.254) (layer F.Cu) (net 12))
 (segment (start 120.396 72.0725) (end 122.555 72.0725) (width 0.254) (layer F.Cu) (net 12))
 (segment (start 114.71 71.15) (end 115.6 71.15) (width 0.254) (layer F.Cu) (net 12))
 (segment (start 115.6 71.15) (end 116.332 71.882) (width 0.254) (layer F.Cu) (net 12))
 (segment (start 119.0625 72.8525) (end 119.0625 71.882) (width 0.254) (layer F.Cu) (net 12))
 (segment (start 116.332 71.882) (end 119.0625 71.882) (width 0.254) (layer F.Cu) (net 12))
 (segment (start 119.0625 71.882) (end 120.2055 71.882) (width 0.254) (layer F.Cu) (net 12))
 (segment (start 98.425 64.77) (end 98.425 64.4525) (width 0.254) (layer F.Cu) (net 2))
 (segment (start 99.695 66.04) (end 98.425 64.77) (width 0.254) (layer F.Cu) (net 2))
 (segment (start 107.98 71.15) (end 105.41 68.58) (width 0.254) (layer F.Cu) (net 2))
 (segment (start 108.81 71.15) (end 107.98 71.15) (width 0.254) (layer F.Cu) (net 2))
 (segment (start 105.41 68.58) (end 100.965 68.58) (width 0.254) (layer F.Cu) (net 2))
 (segment (start 99.695 67.31) (end 99.695 66.04) (width 0.254) (layer F.Cu) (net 2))
 (segment (start 100.965 68.58) (end 99.695 67.31) (width 0.254) (layer F.Cu) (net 2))
 (segment (start 101.6 70.485) (end 103.1875 72.0725) (width 0.381) (layer F.Cu) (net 14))
 (segment (start 100.6475 70.485) (end 101.6 70.485) (width 0.381) (layer F.Cu) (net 14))
 (segment (start 103.1875 72.0725) (end 103.1875 73.9775) (width 0.381) (layer F.Cu) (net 14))
 (segment (start 98.425 66.9925) (end 98.425 68.2625) (width 0.381) (layer F.Cu) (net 14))
 (segment (start 98.425 68.2625) (end 100.6475 70.485) (width 0.381) (layer F.Cu) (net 14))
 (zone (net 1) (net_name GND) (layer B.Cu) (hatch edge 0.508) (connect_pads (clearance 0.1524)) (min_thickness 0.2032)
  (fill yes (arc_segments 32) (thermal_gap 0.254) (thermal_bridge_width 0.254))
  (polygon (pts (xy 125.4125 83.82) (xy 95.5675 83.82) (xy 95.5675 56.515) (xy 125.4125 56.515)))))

